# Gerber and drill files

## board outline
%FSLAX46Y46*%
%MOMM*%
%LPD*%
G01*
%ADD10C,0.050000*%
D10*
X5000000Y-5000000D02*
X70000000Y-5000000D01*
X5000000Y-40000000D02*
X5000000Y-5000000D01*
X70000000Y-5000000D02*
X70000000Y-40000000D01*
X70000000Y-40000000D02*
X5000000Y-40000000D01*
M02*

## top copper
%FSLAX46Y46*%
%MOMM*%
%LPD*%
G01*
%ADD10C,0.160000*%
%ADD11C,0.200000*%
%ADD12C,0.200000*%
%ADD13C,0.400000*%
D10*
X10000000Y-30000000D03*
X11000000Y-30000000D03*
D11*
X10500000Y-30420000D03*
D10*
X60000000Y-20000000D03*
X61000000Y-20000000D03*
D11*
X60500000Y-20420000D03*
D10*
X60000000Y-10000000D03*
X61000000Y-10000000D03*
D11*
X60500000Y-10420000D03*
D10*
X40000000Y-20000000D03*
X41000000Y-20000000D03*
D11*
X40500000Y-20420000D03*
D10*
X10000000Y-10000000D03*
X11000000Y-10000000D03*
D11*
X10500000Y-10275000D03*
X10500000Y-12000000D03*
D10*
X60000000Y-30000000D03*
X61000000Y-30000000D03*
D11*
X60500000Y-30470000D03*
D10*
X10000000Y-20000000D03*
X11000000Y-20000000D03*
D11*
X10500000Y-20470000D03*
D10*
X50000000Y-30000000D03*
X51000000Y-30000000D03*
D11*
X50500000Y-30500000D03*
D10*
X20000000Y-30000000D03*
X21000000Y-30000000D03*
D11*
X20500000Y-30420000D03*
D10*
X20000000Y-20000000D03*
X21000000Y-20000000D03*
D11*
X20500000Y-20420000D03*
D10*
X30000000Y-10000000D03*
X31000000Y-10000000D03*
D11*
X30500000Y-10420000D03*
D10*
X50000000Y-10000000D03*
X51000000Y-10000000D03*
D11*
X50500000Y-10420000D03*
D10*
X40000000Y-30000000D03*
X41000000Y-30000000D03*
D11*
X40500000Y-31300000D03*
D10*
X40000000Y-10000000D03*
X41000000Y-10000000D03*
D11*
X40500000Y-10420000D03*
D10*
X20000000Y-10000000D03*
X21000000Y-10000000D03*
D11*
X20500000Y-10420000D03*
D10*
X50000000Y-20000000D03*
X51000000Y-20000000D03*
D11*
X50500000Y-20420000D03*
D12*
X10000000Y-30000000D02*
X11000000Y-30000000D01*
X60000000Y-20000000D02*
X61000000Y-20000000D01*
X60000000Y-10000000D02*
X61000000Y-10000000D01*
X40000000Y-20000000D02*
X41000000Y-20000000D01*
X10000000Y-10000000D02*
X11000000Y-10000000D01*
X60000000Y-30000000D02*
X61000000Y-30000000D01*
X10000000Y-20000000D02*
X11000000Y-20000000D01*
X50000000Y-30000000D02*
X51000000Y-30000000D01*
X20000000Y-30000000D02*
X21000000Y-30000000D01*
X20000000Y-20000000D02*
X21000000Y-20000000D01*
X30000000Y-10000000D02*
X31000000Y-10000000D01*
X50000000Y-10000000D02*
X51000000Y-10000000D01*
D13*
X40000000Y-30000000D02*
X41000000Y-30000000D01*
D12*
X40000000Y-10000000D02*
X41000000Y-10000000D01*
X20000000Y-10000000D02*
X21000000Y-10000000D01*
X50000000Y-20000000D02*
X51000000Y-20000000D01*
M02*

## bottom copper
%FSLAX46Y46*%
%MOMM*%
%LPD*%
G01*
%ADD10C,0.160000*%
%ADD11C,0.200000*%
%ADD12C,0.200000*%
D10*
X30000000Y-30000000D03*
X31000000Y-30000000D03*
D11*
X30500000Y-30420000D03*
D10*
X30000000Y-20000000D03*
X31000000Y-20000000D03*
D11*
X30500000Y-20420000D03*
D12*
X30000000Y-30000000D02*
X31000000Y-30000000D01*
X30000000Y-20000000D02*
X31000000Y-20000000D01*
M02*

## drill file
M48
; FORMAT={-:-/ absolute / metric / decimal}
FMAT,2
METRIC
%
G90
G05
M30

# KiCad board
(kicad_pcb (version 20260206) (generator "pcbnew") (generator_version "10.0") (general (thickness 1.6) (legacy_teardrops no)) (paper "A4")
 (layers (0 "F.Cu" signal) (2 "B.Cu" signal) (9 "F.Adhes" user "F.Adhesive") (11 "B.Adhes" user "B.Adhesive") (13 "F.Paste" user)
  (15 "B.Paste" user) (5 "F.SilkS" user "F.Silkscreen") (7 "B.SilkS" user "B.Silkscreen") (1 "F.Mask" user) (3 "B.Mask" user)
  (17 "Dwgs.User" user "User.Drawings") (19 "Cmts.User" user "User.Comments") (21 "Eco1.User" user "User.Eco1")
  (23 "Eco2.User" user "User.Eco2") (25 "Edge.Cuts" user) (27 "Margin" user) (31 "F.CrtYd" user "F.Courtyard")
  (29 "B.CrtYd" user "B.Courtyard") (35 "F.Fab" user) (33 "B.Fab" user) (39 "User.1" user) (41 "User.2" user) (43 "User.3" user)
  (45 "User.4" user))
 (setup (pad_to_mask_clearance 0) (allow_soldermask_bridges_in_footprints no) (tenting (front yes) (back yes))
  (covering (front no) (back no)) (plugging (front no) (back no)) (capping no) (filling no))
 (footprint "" (layer "F.Cu") (at 10 30)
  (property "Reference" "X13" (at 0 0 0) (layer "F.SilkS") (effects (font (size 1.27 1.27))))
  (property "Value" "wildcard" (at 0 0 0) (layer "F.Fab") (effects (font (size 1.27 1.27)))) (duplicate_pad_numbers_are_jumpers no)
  (pad "1" smd circle (at 0 0) (size 0.16 0.16) (layers "F.Cu") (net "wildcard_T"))
  (pad "2" smd circle (at 1 0) (size 0.16 0.16) (layers "F.Cu") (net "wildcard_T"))
  (pad "3" smd circle (at 0.5 0.42) (size 0.2 0.2) (layers "F.Cu") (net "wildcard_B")))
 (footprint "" (layer "F.Cu") (at 60 20)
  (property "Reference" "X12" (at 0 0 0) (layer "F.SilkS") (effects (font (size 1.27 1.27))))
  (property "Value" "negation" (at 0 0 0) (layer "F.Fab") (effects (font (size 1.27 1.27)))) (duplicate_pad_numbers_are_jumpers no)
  (pad "1" smd circle (at 0 0) (size 0.16 0.16) (layers "F.Cu") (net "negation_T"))
  (pad "2" smd circle (at 1 0) (size 0.16 0.16) (layers "F.Cu") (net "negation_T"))
  (pad "3" smd circle (at 0.5 0.42) (size 0.2 0.2) (layers "F.Cu") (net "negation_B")))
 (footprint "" (layer "F.Cu") (at 60 10)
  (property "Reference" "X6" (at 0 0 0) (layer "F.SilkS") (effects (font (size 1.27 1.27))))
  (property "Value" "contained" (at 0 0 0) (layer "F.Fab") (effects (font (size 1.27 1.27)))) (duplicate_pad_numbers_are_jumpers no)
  (pad "1" smd circle (at 0 0) (size 0.16 0.16) (layers "F.Cu") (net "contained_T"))
  (pad "2" smd circle (at 1 0) (size 0.16 0.16) (layers "F.Cu") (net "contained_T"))
  (pad "3" smd circle (at 0.5 0.42) (size 0.2 0.2) (layers "F.Cu") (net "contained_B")))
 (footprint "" (layer "F.Cu") (at 40 20)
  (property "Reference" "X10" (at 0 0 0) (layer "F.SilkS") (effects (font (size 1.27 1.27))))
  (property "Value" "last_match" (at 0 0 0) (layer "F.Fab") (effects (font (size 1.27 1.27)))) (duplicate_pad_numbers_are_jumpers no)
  (pad "1" smd circle (at 0 0) (size 0.16 0.16) (layers "F.Cu") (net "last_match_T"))
  (pad "2" smd circle (at 1 0) (size 0.16 0.16) (layers "F.Cu") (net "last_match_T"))
  (pad "3" smd circle (at 0.5 0.42) (size 0.2 0.2) (layers "F.Cu") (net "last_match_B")))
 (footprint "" (layer "F.Cu") (at 10 10)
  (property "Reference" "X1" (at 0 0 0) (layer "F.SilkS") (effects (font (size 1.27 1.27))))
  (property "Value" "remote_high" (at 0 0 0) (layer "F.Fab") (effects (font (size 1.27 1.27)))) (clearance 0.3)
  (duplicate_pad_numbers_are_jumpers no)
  (pad "1" smd circle (at 0 0) (size 0.16 0.16) (layers "F.Cu") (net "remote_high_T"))
  (pad "2" smd circle (at 1 0) (size 0.16 0.16) (layers "F.Cu") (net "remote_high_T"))
  (pad "3" smd circle (at 0.5 0.275) (size 0.2 0.2) (layers "F.Cu") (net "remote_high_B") (clearance 0))
  (pad "4" smd circle (at 0.5 2) (size 0.2 0.2) (layers "F.Cu") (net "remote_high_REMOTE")))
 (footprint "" (layer "F.Cu") (at 60 30)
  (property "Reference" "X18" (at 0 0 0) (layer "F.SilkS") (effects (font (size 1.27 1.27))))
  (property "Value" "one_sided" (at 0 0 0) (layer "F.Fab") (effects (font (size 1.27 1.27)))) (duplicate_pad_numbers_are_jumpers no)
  (pad "1" smd circle (at 0 0) (size 0.16 0.16) (layers "F.Cu") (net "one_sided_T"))
  (pad "2" smd circle (at 1 0) (size 0.16 0.16) (layers "F.Cu") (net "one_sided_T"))
  (pad "3" smd circle (at 0.5 0.47) (size 0.2 0.2) (layers "F.Cu") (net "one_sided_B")))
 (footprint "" (layer "F.Cu") (at 10 20)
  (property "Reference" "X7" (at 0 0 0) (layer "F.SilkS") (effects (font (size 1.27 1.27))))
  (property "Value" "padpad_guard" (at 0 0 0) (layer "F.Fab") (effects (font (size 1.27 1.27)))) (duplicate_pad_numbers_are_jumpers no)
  (pad "1" smd circle (at 0 0) (size 0.16 0.16) (layers "F.Cu") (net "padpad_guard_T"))
  (pad "2" smd circle (at 1 0) (size 0.16 0.16) (layers "F.Cu") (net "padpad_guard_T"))
  (pad "3" smd circle (at 0.5 0.47) (size 0.2 0.2) (layers "F.Cu") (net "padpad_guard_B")))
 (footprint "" (layer "F.Cu") (at 50 30)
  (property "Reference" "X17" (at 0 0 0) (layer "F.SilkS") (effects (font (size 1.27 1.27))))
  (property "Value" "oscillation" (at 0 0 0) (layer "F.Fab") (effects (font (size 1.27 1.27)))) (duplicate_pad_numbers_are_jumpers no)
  (pad "1" smd circle (at 0 0) (size 0.16 0.16) (layers "F.Cu") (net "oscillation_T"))
  (pad "2" smd circle (at 1 0) (size 0.16 0.16) (layers "F.Cu") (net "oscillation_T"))
  (pad "3" smd circle (at 0.5 0.5) (size 0.2 0.2) (layers "F.Cu") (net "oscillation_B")))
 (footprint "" (layer "F.Cu") (at 20 30)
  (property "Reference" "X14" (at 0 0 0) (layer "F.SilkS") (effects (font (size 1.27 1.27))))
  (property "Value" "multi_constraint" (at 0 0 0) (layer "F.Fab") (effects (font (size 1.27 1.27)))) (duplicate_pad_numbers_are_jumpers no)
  (pad "1" smd circle (at 0 0) (size 0.16 0.16) (layers "F.Cu") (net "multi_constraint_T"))
  (pad "2" smd circle (at 1 0) (size 0.16 0.16) (layers "F.Cu") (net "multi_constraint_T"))
  (pad "3" smd circle (at 0.5 0.42) (size 0.2 0.2) (layers "F.Cu") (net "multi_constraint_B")))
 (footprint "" (layer "F.Cu") (at 30 30)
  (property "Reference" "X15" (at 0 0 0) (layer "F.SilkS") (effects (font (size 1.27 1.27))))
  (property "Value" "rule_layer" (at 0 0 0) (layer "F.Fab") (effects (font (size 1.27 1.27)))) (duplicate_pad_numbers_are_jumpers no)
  (pad "1" smd circle (at 0 0) (size 0.16 0.16) (layers "B.Cu") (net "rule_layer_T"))
  (pad "2" smd circle (at 1 0) (size 0.16 0.16) (layers "B.Cu") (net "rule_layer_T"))
  (pad "3" smd circle (at 0.5 0.42) (size 0.2 0.2) (layers "B.Cu") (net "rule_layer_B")))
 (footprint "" (layer "F.Cu") (at 20 20)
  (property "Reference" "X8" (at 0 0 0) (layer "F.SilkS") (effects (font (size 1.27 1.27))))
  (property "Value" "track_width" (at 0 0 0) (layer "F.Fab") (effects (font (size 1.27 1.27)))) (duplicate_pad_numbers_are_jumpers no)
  (pad "1" smd circle (at 0 0) (size 0.16 0.16) (layers "F.Cu") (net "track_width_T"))
  (pad "2" smd circle (at 1 0) (size 0.16 0.16) (layers "F.Cu") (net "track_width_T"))
  (pad "3" smd circle (at 0.5 0.42) (size 0.2 0.2) (layers "F.Cu") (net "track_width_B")))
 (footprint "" (layer "F.Cu") (at 30 10)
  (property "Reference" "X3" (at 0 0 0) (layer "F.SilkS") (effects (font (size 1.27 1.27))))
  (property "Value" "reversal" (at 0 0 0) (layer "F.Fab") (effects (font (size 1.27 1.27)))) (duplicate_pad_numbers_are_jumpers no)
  (pad "1" smd circle (at 0 0) (size 0.16 0.16) (layers "F.Cu") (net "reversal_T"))
  (pad "2" smd circle (at 1 0) (size 0.16 0.16) (layers "F.Cu") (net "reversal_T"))
  (pad "3" smd circle (at 0.5 0.42) (size 0.2 0.2) (layers "F.Cu") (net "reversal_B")))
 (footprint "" (layer "F.Cu") (at 50 10)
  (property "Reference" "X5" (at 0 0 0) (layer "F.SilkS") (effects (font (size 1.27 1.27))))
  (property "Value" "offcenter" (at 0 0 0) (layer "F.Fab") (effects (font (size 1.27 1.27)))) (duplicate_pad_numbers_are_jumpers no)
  (pad "1" smd circle (at 0 0) (size 0.16 0.16) (layers "F.Cu") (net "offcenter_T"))
  (pad "2" smd circle (at 1 0) (size 0.16 0.16) (layers "F.Cu") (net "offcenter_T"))
  (pad "3" smd circle (at 0.5 0.42) (size 0.2 0.2) (layers "F.Cu") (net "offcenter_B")))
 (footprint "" (layer "F.Cu") (at 40 30)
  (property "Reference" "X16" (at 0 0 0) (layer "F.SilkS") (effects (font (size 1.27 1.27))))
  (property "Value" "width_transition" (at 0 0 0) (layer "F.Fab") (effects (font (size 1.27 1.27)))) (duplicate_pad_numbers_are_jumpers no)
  (pad "1" smd circle (at 0 0) (size 0.16 0.16) (layers "F.Cu") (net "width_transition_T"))
  (pad "2" smd circle (at 1 0) (size 0.16 0.16) (layers "F.Cu") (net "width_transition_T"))
  (pad "3" smd circle (at 0.5 1.3) (size 0.2 0.2) (layers "F.Cu") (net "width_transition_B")))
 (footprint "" (layer "F.Cu") (at 30 20)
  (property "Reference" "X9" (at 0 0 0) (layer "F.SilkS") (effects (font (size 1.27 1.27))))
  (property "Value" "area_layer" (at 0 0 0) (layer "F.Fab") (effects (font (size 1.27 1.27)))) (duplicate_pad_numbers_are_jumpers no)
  (pad "1" smd circle (at 0 0) (size 0.16 0.16) (layers "B.Cu") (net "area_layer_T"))
  (pad "2" smd circle (at 1 0) (size 0.16 0.16) (layers "B.Cu") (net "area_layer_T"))
  (pad "3" smd circle (at 0.5 0.42) (size 0.2 0.2) (layers "B.Cu") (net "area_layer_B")))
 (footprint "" (layer "F.Cu") (at 40 10)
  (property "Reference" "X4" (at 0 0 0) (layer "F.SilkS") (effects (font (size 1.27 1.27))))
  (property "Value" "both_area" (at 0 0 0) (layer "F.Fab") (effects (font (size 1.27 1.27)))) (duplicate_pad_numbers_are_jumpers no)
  (pad "1" smd circle (at 0 0) (size 0.16 0.16) (layers "F.Cu") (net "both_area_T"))
  (pad "2" smd circle (at 1 0) (size 0.16 0.16) (layers "F.Cu") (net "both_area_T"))
  (pad "3" smd circle (at 0.5 0.42) (size 0.2 0.2) (layers "F.Cu") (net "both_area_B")))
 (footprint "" (layer "F.Cu") (at 20 10)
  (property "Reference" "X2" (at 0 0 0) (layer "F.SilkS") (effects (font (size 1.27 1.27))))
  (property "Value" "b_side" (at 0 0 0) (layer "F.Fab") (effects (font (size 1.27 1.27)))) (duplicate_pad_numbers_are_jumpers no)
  (pad "1" smd circle (at 0 0) (size 0.16 0.16) (layers "F.Cu") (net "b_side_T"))
  (pad "2" smd circle (at 1 0) (size 0.16 0.16) (layers "F.Cu") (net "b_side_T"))
  (pad "3" smd circle (at 0.5 0.42) (size 0.2 0.2) (layers "F.Cu") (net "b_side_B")))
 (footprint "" (layer "F.Cu") (at 50 20)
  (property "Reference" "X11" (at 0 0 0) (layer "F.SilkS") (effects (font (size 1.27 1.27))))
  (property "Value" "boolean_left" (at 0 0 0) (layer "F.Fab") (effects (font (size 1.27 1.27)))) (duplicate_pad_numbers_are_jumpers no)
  (pad "1" smd circle (at 0 0) (size 0.16 0.16) (layers "F.Cu") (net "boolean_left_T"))
  (pad "2" smd circle (at 1 0) (size 0.16 0.16) (layers "F.Cu") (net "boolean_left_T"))
  (pad "3" smd circle (at 0.5 0.42) (size 0.2 0.2) (layers "F.Cu") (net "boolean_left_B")))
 (gr_line (start 5 5) (end 70 5) (stroke (width 0.05) (type default)) (layer "Edge.Cuts"))
 (gr_line (start 5 40) (end 5 5) (stroke (width 0.05) (type default)) (layer "Edge.Cuts"))
 (gr_line (start 70 5) (end 70 40) (stroke (width 0.05) (type default)) (layer "Edge.Cuts"))
 (gr_line (start 70 40) (end 5 40) (stroke (width 0.05) (type default)) (layer "Edge.Cuts"))
 (segment (start 10 30) (end 11 30) (width 0.2) (layer "F.Cu") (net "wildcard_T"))
 (segment (start 60 20) (end 61 20) (width 0.2) (layer "F.Cu") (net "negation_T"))
 (segment (start 60 10) (end 61 10) (width 0.2) (layer "F.Cu") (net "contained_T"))
 (segment (start 40 20) (end 41 20) (width 0.2) (layer "F.Cu") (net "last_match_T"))
 (segment (start 10 10) (end 11 10) (width 0.2) (layer "F.Cu") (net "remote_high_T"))
 (segment (start 60 30) (end 61 30) (width 0.2) (layer "F.Cu") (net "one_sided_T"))
 (segment (start 10 20) (end 11 20) (width 0.2) (layer "F.Cu") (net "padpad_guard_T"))
 (segment (start 50 30) (end 51 30) (width 0.2) (layer "F.Cu") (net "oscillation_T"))
 (segment (start 20 30) (end 21 30) (width 0.2) (layer "F.Cu") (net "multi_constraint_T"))
 (segment (start 30 30) (end 31 30) (width 0.2) (layer "B.Cu") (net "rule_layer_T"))
 (segment (start 20 20) (end 21 20) (width 0.2) (layer "F.Cu") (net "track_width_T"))
 (segment (start 30 10) (end 31 10) (width 0.2) (layer "F.Cu") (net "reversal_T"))
 (segment (start 50 10) (end 51 10) (width 0.2) (layer "F.Cu") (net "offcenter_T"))
 (segment (start 40 30) (end 41 30) (width 0.4) (layer "F.Cu") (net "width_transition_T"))
 (segment (start 30 20) (end 31 20) (width 0.2) (layer "B.Cu") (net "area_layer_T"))
 (segment (start 40 10) (end 41 10) (width 0.2) (layer "F.Cu") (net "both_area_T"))
 (segment (start 20 10) (end 21 10) (width 0.2) (layer "F.Cu") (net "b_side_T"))
 (segment (start 50 20) (end 51 20) (width 0.2) (layer "F.Cu") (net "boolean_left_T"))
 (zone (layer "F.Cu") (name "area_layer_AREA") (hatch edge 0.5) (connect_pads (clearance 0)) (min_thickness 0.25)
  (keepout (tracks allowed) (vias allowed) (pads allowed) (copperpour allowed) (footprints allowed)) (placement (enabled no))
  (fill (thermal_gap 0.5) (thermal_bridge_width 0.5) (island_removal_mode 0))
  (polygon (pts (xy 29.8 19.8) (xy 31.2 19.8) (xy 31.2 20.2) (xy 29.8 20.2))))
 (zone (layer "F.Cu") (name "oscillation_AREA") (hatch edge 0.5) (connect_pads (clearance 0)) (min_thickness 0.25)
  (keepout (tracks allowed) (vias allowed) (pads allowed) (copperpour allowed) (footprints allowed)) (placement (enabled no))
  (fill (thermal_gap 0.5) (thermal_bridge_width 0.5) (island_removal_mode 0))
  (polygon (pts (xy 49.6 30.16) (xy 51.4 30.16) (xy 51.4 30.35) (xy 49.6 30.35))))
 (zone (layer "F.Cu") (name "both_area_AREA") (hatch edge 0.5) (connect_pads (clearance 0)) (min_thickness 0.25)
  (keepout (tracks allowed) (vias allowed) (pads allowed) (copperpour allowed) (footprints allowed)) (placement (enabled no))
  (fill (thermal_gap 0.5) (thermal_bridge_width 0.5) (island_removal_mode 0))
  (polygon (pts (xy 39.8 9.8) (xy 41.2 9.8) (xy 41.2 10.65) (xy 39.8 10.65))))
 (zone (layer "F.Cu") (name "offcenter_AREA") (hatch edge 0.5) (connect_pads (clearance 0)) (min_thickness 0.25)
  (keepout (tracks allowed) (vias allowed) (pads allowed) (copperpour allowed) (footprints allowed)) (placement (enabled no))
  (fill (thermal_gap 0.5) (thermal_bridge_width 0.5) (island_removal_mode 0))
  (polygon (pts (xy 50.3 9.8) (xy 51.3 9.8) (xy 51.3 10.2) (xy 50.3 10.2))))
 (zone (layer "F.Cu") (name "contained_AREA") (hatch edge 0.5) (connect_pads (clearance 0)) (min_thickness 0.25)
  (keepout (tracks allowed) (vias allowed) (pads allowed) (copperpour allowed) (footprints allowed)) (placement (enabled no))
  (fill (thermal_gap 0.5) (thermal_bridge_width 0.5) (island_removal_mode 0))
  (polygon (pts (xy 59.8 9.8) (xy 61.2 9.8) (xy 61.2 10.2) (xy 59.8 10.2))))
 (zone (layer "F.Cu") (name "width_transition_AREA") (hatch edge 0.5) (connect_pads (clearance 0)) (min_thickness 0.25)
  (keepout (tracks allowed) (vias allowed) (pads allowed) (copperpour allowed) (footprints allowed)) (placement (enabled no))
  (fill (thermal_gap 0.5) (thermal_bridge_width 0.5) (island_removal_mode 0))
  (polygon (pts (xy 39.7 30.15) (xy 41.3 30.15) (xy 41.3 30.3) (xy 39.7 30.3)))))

